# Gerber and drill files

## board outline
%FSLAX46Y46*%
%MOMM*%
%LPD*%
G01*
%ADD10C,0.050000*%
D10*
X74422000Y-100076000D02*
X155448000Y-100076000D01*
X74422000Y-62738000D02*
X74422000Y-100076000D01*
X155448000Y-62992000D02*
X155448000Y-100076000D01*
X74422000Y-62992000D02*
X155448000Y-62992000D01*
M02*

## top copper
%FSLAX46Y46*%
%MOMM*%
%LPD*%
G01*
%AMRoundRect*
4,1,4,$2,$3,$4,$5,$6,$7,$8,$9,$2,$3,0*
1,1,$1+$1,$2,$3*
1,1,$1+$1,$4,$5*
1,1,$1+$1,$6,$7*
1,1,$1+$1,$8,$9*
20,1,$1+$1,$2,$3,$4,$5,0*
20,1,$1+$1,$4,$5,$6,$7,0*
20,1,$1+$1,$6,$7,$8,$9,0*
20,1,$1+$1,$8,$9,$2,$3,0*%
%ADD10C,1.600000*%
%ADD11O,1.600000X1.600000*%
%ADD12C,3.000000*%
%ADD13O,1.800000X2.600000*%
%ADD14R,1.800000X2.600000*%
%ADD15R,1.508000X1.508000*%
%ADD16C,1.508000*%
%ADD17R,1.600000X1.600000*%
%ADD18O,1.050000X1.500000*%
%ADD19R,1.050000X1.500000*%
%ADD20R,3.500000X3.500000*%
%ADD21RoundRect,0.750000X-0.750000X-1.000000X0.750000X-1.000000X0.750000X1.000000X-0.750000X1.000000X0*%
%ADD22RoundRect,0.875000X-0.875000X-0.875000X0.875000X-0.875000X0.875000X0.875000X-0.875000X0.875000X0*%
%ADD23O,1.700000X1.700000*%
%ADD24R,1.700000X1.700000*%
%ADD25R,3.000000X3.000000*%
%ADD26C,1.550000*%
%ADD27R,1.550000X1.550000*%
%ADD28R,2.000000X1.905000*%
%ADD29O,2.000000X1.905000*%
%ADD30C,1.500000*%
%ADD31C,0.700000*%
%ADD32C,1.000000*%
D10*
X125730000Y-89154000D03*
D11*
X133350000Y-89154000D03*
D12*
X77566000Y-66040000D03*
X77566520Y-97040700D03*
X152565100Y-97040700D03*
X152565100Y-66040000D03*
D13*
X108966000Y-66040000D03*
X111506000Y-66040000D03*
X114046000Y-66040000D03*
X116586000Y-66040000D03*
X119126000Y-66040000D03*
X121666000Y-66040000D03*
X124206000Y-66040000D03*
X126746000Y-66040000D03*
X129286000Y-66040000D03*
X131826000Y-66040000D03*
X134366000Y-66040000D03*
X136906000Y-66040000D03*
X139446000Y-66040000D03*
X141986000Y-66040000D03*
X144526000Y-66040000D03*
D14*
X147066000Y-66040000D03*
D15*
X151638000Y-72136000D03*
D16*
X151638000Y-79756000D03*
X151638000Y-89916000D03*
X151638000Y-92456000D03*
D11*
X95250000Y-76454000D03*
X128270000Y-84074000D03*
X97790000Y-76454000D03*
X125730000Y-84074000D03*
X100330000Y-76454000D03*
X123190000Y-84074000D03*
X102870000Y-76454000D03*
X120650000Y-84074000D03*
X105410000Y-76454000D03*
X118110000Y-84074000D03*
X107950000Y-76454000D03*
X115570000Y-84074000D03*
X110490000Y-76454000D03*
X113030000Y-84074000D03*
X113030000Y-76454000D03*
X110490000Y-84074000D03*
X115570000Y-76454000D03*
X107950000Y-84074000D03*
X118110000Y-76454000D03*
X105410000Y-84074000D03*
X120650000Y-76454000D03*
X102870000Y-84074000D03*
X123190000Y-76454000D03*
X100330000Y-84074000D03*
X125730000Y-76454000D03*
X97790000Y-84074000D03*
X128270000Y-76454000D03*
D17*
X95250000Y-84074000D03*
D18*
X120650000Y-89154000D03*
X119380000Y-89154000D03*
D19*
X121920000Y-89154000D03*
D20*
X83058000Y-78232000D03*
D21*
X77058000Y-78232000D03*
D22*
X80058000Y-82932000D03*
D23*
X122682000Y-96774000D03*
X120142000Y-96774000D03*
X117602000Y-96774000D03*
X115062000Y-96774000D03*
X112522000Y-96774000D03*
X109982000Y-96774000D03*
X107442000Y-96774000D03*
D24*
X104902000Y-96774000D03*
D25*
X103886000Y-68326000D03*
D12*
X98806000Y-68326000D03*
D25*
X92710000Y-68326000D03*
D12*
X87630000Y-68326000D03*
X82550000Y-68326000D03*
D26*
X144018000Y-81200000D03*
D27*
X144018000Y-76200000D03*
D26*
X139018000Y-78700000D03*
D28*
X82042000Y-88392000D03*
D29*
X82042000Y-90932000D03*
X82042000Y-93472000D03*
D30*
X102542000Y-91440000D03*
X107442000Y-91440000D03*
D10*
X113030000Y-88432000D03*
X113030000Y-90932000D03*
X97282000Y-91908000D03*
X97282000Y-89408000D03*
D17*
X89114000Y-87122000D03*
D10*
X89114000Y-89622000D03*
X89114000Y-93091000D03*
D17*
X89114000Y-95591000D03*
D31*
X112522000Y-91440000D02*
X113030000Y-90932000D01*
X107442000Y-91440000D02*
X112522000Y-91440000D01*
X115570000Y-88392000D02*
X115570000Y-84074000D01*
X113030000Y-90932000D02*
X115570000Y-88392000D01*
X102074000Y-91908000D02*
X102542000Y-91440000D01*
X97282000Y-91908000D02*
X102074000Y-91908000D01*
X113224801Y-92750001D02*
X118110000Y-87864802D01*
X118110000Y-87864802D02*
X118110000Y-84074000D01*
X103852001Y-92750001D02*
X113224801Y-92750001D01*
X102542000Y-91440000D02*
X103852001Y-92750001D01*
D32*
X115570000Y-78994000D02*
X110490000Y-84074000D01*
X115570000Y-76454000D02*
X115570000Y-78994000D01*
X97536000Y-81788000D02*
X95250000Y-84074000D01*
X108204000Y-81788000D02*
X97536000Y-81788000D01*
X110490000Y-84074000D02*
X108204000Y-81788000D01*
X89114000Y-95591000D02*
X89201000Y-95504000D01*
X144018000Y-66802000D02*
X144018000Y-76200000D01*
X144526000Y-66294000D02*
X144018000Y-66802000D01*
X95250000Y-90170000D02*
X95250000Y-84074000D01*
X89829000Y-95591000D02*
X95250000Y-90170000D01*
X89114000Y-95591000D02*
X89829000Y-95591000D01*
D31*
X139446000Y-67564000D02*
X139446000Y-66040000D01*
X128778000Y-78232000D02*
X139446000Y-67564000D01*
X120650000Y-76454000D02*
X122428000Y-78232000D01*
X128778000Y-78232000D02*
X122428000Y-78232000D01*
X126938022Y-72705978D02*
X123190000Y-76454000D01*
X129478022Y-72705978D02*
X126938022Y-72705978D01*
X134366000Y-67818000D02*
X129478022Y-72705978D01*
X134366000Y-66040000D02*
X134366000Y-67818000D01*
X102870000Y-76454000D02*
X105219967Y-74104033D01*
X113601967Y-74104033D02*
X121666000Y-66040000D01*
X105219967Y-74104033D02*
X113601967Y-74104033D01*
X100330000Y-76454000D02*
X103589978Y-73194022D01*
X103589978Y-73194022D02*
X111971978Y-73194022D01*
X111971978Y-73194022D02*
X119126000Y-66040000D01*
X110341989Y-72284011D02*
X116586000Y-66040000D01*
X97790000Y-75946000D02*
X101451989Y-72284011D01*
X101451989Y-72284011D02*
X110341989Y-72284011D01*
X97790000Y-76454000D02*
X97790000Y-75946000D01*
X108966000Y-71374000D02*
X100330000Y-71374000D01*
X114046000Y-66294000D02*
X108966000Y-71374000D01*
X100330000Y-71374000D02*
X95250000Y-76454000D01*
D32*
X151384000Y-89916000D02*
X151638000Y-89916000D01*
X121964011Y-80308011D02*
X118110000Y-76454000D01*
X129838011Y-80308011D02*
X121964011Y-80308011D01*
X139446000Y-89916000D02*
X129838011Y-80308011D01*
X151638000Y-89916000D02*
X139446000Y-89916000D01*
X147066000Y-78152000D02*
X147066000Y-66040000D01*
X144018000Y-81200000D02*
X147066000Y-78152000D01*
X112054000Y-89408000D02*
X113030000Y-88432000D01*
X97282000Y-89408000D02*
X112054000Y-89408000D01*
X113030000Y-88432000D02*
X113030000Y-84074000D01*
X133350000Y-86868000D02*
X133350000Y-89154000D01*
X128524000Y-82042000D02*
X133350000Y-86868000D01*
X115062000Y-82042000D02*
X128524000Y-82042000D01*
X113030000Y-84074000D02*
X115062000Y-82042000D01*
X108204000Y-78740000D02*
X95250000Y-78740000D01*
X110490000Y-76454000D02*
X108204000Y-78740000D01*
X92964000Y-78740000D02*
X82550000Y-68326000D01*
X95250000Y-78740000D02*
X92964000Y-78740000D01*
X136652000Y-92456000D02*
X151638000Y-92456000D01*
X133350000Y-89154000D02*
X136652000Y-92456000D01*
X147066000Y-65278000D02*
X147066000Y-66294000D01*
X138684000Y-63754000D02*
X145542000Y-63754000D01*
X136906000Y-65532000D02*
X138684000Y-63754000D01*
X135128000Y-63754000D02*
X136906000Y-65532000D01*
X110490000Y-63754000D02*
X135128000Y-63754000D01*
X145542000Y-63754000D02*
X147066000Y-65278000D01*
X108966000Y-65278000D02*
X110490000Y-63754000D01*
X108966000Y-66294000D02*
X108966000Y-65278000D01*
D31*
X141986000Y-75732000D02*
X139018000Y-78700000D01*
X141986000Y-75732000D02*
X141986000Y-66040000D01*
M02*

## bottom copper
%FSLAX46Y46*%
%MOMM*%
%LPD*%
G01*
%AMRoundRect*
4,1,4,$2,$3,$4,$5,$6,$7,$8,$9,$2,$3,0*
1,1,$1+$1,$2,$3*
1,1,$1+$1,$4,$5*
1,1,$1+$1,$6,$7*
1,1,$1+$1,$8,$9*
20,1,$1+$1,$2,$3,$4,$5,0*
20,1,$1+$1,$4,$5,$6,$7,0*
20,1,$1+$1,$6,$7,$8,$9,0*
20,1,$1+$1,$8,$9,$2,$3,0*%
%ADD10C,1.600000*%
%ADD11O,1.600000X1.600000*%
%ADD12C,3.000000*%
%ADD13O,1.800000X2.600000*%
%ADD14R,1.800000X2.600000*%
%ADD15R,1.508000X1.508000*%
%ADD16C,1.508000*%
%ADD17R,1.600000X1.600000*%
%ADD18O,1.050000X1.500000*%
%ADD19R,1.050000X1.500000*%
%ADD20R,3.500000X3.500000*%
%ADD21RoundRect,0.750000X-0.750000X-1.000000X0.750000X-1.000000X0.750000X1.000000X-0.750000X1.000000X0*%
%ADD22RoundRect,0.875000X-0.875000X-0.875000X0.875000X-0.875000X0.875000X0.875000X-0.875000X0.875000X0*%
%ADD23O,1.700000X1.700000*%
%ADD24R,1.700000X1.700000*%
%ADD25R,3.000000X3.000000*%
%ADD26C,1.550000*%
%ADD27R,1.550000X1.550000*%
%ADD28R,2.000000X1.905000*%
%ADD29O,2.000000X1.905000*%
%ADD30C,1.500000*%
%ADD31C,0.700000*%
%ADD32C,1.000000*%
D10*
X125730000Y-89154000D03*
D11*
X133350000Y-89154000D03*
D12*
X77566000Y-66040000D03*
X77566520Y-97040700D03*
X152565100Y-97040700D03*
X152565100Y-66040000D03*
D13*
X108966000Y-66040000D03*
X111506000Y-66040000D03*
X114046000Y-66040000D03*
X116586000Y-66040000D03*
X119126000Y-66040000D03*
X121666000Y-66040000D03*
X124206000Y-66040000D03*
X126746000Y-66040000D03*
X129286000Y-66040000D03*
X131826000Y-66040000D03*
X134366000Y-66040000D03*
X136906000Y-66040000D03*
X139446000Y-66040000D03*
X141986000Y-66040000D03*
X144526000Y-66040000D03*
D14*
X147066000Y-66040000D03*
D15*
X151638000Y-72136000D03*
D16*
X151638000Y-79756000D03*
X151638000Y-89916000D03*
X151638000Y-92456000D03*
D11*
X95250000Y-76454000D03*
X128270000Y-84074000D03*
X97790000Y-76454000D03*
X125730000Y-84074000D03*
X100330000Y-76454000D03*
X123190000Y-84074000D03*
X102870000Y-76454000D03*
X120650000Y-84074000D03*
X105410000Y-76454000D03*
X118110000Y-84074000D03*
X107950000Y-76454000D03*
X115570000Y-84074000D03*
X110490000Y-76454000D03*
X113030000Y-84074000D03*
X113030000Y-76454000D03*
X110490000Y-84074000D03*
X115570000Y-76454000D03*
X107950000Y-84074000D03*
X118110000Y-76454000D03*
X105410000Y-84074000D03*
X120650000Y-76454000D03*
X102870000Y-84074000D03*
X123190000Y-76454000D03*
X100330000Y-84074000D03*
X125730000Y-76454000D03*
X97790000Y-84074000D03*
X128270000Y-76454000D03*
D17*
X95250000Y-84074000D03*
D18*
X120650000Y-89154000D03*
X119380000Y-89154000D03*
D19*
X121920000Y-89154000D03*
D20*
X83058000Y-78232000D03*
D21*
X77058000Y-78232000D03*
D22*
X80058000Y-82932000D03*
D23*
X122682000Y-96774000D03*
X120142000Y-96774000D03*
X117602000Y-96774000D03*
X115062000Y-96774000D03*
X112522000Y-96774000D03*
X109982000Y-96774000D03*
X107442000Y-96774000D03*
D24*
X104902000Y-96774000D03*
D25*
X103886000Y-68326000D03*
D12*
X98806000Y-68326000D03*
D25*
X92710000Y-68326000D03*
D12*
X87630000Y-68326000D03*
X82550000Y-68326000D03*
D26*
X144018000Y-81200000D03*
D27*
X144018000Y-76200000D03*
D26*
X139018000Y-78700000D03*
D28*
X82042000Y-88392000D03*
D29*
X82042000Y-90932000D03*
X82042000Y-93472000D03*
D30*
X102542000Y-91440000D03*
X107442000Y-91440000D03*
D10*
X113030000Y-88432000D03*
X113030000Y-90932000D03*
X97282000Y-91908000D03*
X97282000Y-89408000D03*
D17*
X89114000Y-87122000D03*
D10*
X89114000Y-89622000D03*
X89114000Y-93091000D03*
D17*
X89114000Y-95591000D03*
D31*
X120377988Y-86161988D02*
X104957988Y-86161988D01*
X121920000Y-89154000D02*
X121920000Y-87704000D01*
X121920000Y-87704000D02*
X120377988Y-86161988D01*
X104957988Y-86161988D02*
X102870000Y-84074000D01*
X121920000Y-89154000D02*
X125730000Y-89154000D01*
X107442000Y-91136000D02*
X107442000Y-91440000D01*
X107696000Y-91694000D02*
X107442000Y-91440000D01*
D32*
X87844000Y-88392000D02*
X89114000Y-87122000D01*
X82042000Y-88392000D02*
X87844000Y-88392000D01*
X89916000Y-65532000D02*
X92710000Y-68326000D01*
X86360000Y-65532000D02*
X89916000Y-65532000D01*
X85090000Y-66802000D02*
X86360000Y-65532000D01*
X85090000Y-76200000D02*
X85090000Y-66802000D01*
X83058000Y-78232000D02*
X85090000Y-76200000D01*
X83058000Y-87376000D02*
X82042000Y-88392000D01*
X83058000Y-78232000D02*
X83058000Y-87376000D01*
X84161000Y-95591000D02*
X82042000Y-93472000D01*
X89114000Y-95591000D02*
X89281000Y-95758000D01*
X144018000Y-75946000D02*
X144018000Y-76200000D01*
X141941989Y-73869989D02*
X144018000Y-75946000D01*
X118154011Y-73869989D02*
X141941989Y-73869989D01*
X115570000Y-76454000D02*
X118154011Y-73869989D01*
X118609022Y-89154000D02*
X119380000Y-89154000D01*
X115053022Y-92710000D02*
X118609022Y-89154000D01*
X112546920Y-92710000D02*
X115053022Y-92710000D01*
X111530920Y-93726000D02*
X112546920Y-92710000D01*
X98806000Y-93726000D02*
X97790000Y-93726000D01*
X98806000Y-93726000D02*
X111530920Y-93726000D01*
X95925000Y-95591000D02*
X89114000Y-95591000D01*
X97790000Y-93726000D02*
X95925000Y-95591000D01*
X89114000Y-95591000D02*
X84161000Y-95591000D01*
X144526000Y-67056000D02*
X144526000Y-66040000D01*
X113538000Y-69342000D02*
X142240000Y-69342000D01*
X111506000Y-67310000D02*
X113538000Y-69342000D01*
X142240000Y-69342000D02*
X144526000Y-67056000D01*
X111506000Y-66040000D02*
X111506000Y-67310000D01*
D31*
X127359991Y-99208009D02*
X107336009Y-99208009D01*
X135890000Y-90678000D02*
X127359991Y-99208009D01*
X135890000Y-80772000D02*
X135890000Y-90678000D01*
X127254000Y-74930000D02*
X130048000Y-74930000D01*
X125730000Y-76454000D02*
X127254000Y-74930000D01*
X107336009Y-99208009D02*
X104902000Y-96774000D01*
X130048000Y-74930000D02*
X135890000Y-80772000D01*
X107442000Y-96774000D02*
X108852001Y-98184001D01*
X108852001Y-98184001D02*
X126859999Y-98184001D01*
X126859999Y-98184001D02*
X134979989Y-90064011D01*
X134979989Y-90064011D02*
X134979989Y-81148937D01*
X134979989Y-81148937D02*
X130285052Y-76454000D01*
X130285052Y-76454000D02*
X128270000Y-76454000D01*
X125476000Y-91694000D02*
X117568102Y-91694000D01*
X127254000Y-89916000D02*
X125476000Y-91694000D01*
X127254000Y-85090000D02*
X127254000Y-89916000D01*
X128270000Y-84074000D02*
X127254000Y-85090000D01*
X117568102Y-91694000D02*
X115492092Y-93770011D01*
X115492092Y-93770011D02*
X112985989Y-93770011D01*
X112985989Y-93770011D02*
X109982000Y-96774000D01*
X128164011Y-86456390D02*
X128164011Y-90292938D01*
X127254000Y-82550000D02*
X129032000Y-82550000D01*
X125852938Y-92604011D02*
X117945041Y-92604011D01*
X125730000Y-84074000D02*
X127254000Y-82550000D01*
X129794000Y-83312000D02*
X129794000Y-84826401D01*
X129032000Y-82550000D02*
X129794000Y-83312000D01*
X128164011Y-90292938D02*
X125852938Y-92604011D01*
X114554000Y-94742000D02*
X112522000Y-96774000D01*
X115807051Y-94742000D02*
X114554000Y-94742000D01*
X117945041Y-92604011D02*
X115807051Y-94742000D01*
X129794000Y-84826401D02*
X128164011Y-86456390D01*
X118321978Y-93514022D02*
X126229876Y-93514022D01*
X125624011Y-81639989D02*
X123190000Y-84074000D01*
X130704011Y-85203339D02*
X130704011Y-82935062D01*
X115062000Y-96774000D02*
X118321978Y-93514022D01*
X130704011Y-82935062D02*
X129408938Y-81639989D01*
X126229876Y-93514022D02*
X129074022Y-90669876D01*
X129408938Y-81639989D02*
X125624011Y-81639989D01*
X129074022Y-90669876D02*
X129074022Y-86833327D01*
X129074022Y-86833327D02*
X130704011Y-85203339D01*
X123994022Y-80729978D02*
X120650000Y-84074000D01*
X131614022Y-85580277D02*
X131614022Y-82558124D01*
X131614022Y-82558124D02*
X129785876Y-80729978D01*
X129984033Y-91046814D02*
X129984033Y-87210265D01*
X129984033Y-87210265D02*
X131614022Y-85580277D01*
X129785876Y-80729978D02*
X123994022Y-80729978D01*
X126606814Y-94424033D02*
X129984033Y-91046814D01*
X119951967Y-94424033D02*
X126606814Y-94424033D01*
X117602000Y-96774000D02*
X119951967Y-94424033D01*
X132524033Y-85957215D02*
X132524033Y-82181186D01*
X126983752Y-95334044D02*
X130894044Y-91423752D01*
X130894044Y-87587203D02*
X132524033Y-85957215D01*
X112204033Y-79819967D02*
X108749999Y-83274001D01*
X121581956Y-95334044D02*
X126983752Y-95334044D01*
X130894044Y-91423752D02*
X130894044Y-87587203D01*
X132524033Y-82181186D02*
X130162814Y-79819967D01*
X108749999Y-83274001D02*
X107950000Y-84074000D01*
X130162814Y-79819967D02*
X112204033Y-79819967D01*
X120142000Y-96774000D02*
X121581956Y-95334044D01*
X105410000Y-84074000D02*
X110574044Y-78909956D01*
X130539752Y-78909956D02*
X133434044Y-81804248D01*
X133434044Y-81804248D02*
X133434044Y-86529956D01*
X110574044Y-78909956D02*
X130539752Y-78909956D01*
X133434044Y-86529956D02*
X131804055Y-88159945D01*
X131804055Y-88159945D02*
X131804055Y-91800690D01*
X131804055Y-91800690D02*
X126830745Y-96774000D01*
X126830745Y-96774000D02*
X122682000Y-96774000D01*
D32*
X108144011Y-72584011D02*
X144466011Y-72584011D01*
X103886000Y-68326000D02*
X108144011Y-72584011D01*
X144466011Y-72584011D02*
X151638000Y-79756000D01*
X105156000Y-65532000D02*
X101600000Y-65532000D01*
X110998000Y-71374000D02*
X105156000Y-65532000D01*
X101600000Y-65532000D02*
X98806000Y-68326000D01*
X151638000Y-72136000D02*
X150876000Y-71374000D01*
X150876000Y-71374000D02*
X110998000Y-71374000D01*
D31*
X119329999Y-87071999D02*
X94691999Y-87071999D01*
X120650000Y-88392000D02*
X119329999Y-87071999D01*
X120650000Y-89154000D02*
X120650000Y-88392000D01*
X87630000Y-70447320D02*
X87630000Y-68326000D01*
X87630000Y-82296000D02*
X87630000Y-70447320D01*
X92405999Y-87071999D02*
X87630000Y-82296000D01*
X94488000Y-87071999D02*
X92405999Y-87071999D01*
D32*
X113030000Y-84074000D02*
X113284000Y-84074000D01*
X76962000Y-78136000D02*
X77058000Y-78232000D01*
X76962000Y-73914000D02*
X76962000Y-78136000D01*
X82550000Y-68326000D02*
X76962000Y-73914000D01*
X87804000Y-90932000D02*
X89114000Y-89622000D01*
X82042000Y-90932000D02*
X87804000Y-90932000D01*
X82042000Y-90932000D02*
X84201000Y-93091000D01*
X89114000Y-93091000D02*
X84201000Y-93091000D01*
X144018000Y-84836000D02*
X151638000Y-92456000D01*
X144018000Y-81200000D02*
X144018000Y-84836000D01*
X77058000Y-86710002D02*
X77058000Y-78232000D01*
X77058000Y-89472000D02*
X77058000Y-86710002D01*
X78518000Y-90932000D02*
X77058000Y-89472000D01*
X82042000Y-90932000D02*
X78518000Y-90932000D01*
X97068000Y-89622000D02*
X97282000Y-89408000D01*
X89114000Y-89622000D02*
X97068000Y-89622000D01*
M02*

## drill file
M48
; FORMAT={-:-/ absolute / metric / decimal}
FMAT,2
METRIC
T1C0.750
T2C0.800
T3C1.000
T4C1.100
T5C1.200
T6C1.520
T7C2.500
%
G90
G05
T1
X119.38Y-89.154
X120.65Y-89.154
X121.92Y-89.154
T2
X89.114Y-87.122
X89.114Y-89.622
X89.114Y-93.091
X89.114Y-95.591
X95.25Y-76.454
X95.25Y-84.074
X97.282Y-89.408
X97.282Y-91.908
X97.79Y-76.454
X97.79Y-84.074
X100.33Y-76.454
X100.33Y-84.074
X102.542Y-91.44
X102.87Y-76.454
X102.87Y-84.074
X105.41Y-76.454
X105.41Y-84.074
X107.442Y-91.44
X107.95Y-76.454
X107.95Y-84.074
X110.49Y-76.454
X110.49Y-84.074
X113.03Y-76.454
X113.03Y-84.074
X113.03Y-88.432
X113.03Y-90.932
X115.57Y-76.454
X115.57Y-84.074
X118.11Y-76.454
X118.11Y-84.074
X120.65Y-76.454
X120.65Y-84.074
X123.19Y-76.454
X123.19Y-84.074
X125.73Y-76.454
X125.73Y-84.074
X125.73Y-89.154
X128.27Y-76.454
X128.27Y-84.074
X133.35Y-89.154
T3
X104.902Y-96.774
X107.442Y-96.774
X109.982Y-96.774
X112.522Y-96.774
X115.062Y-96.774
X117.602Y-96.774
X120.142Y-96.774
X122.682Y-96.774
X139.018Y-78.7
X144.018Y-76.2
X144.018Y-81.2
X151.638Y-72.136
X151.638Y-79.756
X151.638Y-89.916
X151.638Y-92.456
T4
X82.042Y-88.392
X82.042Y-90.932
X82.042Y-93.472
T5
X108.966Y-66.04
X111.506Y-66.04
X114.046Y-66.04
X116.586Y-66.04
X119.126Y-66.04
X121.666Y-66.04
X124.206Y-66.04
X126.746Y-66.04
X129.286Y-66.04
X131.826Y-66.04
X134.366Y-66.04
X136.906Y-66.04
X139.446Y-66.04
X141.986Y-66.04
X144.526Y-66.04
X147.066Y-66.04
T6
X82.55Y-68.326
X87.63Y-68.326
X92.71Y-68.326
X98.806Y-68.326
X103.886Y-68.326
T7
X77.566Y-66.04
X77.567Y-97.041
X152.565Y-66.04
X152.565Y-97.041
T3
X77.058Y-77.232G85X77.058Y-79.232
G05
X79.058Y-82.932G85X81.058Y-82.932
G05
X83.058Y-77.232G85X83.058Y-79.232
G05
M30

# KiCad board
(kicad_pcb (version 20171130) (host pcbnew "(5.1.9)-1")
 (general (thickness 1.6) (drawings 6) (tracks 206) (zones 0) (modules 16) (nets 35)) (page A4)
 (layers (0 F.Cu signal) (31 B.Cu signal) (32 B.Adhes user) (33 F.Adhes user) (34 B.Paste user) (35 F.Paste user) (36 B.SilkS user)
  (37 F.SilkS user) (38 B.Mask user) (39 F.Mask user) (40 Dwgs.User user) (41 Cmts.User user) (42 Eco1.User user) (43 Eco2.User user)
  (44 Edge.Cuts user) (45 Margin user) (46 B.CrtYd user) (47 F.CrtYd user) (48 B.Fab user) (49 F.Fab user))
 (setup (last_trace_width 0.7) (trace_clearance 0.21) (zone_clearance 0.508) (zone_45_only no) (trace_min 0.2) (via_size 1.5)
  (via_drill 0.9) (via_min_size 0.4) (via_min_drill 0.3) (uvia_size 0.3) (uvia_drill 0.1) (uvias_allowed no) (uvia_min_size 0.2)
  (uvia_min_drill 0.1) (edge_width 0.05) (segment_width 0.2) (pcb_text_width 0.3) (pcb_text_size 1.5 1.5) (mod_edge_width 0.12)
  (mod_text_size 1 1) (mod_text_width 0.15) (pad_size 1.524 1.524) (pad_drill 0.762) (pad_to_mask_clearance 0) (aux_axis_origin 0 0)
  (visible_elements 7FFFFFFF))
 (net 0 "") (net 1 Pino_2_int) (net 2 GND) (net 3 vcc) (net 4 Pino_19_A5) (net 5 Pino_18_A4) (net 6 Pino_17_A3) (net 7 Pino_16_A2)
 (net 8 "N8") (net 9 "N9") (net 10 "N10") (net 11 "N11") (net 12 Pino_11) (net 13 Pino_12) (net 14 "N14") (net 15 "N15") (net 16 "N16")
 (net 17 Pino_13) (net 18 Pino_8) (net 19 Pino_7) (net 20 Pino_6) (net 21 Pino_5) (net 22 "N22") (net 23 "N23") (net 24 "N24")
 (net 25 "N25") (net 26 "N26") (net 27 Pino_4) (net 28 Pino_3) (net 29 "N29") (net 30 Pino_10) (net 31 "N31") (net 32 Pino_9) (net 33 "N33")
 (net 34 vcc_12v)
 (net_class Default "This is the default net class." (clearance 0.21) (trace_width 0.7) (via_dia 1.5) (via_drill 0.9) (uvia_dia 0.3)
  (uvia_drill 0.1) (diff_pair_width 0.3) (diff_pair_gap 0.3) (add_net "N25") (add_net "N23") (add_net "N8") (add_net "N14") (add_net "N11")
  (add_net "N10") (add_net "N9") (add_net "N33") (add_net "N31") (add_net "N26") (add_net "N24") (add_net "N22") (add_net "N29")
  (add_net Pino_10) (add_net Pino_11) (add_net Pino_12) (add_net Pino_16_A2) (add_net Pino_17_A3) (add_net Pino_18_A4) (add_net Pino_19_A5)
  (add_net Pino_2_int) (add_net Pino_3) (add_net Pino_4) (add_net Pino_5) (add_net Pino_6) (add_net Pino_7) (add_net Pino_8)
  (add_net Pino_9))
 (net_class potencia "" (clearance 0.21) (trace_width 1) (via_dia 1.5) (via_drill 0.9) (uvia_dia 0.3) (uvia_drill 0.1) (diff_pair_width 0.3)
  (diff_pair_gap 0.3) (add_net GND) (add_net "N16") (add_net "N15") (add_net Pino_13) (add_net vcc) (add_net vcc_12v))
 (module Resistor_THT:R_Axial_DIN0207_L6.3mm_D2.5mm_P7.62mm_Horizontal (layer F.Cu) (at 125.73 89.154)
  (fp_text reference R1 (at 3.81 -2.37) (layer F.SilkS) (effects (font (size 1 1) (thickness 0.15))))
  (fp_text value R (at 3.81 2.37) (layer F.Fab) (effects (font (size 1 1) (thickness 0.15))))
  (pad 1 thru_hole circle (at 0 0) (size 1.6 1.6) (drill 0.8) (layers *.Cu *.Mask) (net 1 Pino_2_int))
  (pad 2 thru_hole oval (at 7.62 0) (size 1.6 1.6) (drill 0.8) (layers *.Cu *.Mask) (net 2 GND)))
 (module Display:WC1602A (layer B.Cu) (at 147.066 66.04 180)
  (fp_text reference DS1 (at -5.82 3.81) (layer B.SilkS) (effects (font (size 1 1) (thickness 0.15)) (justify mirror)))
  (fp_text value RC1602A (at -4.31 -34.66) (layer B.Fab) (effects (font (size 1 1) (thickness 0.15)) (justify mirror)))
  (pad "" thru_hole circle (at 69.5 0 180) (size 3 3) (drill 2.5) (layers *.Cu *.Mask))
  (pad "" thru_hole circle (at 69.49948 -31.0007 180) (size 3 3) (drill 2.5) (layers *.Cu *.Mask))
  (pad "" thru_hole circle (at -5.4991 -31.0007 180) (size 3 3) (drill 2.5) (layers *.Cu *.Mask))
  (pad "" thru_hole circle (at -5.4991 0 180) (size 3 3) (drill 2.5) (layers *.Cu *.Mask))
  (pad 16 thru_hole oval (at 38.1 0 180) (size 1.8 2.6) (drill 1.2) (layers *.Cu *.Mask) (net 2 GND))
  (pad 15 thru_hole oval (at 35.56 0 180) (size 1.8 2.6) (drill 1.2) (layers *.Cu *.Mask) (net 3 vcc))
  (pad 14 thru_hole oval (at 33.02 0 180) (size 1.8 2.6) (drill 1.2) (layers *.Cu *.Mask) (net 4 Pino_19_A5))
  (pad 13 thru_hole oval (at 30.48 0 180) (size 1.8 2.6) (drill 1.2) (layers *.Cu *.Mask) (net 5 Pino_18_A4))
  (pad 12 thru_hole oval (at 27.94 0 180) (size 1.8 2.6) (drill 1.2) (layers *.Cu *.Mask) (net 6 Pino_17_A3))
  (pad 11 thru_hole oval (at 25.4 0 180) (size 1.8 2.6) (drill 1.2) (layers *.Cu *.Mask) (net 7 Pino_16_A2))
  (pad 10 thru_hole oval (at 22.86 0 180) (size 1.8 2.6) (drill 1.2) (layers *.Cu *.Mask) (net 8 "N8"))
  (pad 9 thru_hole oval (at 20.32 0 180) (size 1.8 2.6) (drill 1.2) (layers *.Cu *.Mask) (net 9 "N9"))
  (pad 8 thru_hole oval (at 17.78 0 180) (size 1.8 2.6) (drill 1.2) (layers *.Cu *.Mask) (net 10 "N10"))
  (pad 7 thru_hole oval (at 15.24 0 180) (size 1.8 2.6) (drill 1.2) (layers *.Cu *.Mask) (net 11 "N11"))
  (pad 6 thru_hole oval (at 12.7 0 180) (size 1.8 2.6) (drill 1.2) (layers *.Cu *.Mask) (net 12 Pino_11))
  (pad 5 thru_hole oval (at 10.16 0 180) (size 1.8 2.6) (drill 1.2) (layers *.Cu *.Mask) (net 2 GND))
  (pad 4 thru_hole oval (at 7.62 0 180) (size 1.8 2.6) (drill 1.2) (layers *.Cu *.Mask) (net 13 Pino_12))
  (pad 3 thru_hole oval (at 5.08 0 180) (size 1.8 2.6) (drill 1.2) (layers *.Cu *.Mask) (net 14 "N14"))
  (pad 2 thru_hole oval (at 2.54 0 180) (size 1.8 2.6) (drill 1.2) (layers *.Cu *.Mask) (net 3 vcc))
  (pad 1 thru_hole rect (at 0 0 180) (size 1.8 2.6) (drill 1.2) (layers *.Cu *.Mask) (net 2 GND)))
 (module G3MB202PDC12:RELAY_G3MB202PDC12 (layer F.Cu) (at 150.238 82.296 270)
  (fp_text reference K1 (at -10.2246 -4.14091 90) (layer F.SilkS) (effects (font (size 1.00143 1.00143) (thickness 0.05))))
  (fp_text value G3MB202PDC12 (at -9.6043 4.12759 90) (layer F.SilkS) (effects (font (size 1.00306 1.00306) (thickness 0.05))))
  (pad 1 thru_hole rect (at -10.16 -1.4 90) (size 1.508 1.508) (drill 1) (layers *.Cu *.Mask) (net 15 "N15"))
  (pad 2 thru_hole circle (at -2.54 -1.4 90) (size 1.508 1.508) (drill 1) (layers *.Cu *.Mask) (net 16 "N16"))
  (pad 3 thru_hole circle (at 7.62 -1.4 90) (size 1.508 1.508) (drill 1) (layers *.Cu *.Mask) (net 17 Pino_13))
  (pad 4 thru_hole circle (at 10.16 -1.4 90) (size 1.508 1.508) (drill 1) (layers *.Cu *.Mask) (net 2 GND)))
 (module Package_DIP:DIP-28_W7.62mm (layer F.Cu) (at 95.25 84.074 90)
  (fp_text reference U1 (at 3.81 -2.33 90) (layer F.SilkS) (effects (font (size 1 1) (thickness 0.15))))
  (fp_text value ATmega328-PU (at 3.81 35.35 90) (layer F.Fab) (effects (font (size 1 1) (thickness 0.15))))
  (pad 28 thru_hole oval (at 7.62 0 90) (size 1.6 1.6) (drill 0.8) (layers *.Cu *.Mask) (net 4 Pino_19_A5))
  (pad 14 thru_hole oval (at 0 33.02 90) (size 1.6 1.6) (drill 0.8) (layers *.Cu *.Mask) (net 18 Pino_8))
  (pad 27 thru_hole oval (at 7.62 2.54 90) (size 1.6 1.6) (drill 0.8) (layers *.Cu *.Mask) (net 5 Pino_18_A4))
  (pad 13 thru_hole oval (at 0 30.48 90) (size 1.6 1.6) (drill 0.8) (layers *.Cu *.Mask) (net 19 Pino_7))
  (pad 26 thru_hole oval (at 7.62 5.08 90) (size 1.6 1.6) (drill 0.8) (layers *.Cu *.Mask) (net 6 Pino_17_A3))
  (pad 12 thru_hole oval (at 0 27.94 90) (size 1.6 1.6) (drill 0.8) (layers *.Cu *.Mask) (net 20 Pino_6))
  (pad 25 thru_hole oval (at 7.62 7.62 90) (size 1.6 1.6) (drill 0.8) (layers *.Cu *.Mask) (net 7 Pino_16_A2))
  (pad 11 thru_hole oval (at 0 25.4 90) (size 1.6 1.6) (drill 0.8) (layers *.Cu *.Mask) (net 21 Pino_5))
  (pad 24 thru_hole oval (at 7.62 10.16 90) (size 1.6 1.6) (drill 0.8) (layers *.Cu *.Mask) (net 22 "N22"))
  (pad 10 thru_hole oval (at 0 22.86 90) (size 1.6 1.6) (drill 0.8) (layers *.Cu *.Mask) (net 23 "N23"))
  (pad 23 thru_hole oval (at 7.62 12.7 90) (size 1.6 1.6) (drill 0.8) (layers *.Cu *.Mask) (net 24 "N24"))
  (pad 9 thru_hole oval (at 0 20.32 90) (size 1.6 1.6) (drill 0.8) (layers *.Cu *.Mask) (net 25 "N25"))
  (pad 22 thru_hole oval (at 7.62 15.24 90) (size 1.6 1.6) (drill 0.8) (layers *.Cu *.Mask) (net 2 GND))
  (pad 8 thru_hole oval (at 0 17.78 90) (size 1.6 1.6) (drill 0.8) (layers *.Cu *.Mask) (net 2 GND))
  (pad 21 thru_hole oval (at 7.62 17.78 90) (size 1.6 1.6) (drill 0.8) (layers *.Cu *.Mask) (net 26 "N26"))
  (pad 7 thru_hole oval (at 0 15.24 90) (size 1.6 1.6) (drill 0.8) (layers *.Cu *.Mask) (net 3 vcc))
  (pad 20 thru_hole oval (at 7.62 20.32 90) (size 1.6 1.6) (drill 0.8) (layers *.Cu *.Mask) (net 3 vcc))
  (pad 6 thru_hole oval (at 0 12.7 90) (size 1.6 1.6) (drill 0.8) (layers *.Cu *.Mask) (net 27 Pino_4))
  (pad 19 thru_hole oval (at 7.62 22.86 90) (size 1.6 1.6) (drill 0.8) (layers *.Cu *.Mask) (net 17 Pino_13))
  (pad 5 thru_hole oval (at 0 10.16 90) (size 1.6 1.6) (drill 0.8) (layers *.Cu *.Mask) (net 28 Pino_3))
  (pad 18 thru_hole oval (at 7.62 25.4 90) (size 1.6 1.6) (drill 0.8) (layers *.Cu *.Mask) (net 13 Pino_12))
  (pad 4 thru_hole oval (at 0 7.62 90) (size 1.6 1.6) (drill 0.8) (layers *.Cu *.Mask) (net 1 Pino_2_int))
  (pad 17 thru_hole oval (at 7.62 27.94 90) (size 1.6 1.6) (drill 0.8) (layers *.Cu *.Mask) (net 12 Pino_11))
  (pad 3 thru_hole oval (at 0 5.08 90) (size 1.6 1.6) (drill 0.8) (layers *.Cu *.Mask) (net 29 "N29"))
  (pad 16 thru_hole oval (at 7.62 30.48 90) (size 1.6 1.6) (drill 0.8) (layers *.Cu *.Mask) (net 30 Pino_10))
  (pad 2 thru_hole oval (at 0 2.54 90) (size 1.6 1.6) (drill 0.8) (layers *.Cu *.Mask) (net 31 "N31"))
  (pad 15 thru_hole oval (at 7.62 33.02 90) (size 1.6 1.6) (drill 0.8) (layers *.Cu *.Mask) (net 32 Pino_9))
  (pad 1 thru_hole rect (at 0 0 90) (size 1.6 1.6) (drill 0.8) (layers *.Cu *.Mask) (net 3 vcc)))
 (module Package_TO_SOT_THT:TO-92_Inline (layer F.Cu) (at 121.92 89.154 180)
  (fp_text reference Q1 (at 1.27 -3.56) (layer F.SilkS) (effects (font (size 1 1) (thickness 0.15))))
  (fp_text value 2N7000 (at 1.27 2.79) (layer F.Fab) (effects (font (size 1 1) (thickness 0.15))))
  (pad 2 thru_hole oval (at 1.27 0 180) (size 1.05 1.5) (drill 0.75) (layers *.Cu *.Mask) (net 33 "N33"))
  (pad 3 thru_hole oval (at 2.54 0 180) (size 1.05 1.5) (drill 0.75) (layers *.Cu *.Mask) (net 3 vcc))
  (pad 1 thru_hole rect (at 0 0 180) (size 1.05 1.5) (drill 0.75) (layers *.Cu *.Mask) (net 1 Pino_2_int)))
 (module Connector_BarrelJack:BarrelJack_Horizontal (layer F.Cu) (at 83.058 78.232)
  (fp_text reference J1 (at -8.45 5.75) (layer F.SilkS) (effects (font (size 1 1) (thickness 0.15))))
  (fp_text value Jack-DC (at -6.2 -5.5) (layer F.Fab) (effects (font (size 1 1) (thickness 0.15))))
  (pad 1 thru_hole rect (at 0 0) (size 3.5 3.5) (drill oval 1 3) (layers *.Cu *.Mask) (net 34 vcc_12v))
  (pad 2 thru_hole roundrect (at -6 0) (size 3 3.5) (drill oval 1 3) (layers *.Cu *.Mask) (roundrect_rratio 0.25) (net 2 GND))
  (pad 3 thru_hole roundrect (at -3 4.7) (size 3.5 3.5) (drill oval 3 1) (layers *.Cu *.Mask) (roundrect_rratio 0.25)))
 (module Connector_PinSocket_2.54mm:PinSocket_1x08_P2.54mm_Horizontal (layer F.Cu) (at 104.902 96.774 90)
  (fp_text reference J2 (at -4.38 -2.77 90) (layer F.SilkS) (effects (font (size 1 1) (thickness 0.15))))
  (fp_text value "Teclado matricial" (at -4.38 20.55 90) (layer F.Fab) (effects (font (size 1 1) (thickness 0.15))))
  (pad 8 thru_hole oval (at 0 17.78 90) (size 1.7 1.7) (drill 1) (layers *.Cu *.Mask) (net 28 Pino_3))
  (pad 7 thru_hole oval (at 0 15.24 90) (size 1.7 1.7) (drill 1) (layers *.Cu *.Mask) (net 27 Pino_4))
  (pad 6 thru_hole oval (at 0 12.7 90) (size 1.7 1.7) (drill 1) (layers *.Cu *.Mask) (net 21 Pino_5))
  (pad 5 thru_hole oval (at 0 10.16 90) (size 1.7 1.7) (drill 1) (layers *.Cu *.Mask) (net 20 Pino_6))
  (pad 4 thru_hole oval (at 0 7.62 90) (size 1.7 1.7) (drill 1) (layers *.Cu *.Mask) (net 19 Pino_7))
  (pad 3 thru_hole oval (at 0 5.08 90) (size 1.7 1.7) (drill 1) (layers *.Cu *.Mask) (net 18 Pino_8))
  (pad 2 thru_hole oval (at 0 2.54 90) (size 1.7 1.7) (drill 1) (layers *.Cu *.Mask) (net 32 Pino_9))
  (pad 1 thru_hole rect (at 0 0 90) (size 1.7 1.7) (drill 1) (layers *.Cu *.Mask) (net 30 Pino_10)))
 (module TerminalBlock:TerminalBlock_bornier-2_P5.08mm (layer F.Cu) (at 103.886 68.326 180)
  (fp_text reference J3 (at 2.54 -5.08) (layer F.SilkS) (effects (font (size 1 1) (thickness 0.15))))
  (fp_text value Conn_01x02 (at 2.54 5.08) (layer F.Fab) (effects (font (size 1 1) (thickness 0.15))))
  (pad 1 thru_hole rect (at 0 0 180) (size 3 3) (drill 1.52) (layers *.Cu *.Mask) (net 16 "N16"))
  (pad 2 thru_hole circle (at 5.08 0 180) (size 3 3) (drill 1.52) (layers *.Cu *.Mask) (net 15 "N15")))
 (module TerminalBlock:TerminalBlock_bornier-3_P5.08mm (layer F.Cu) (at 92.71 68.326 180)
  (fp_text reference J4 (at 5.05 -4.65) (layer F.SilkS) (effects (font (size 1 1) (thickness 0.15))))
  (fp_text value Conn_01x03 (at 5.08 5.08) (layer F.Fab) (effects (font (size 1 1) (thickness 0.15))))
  (pad 1 thru_hole rect (at 0 0 180) (size 3 3) (drill 1.52) (layers *.Cu *.Mask) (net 34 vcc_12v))
  (pad 2 thru_hole circle (at 5.08 0 180) (size 3 3) (drill 1.52) (layers *.Cu *.Mask) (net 33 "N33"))
  (pad 3 thru_hole circle (at 10.16 0 180) (size 3 3) (drill 1.52) (layers *.Cu *.Mask) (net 2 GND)))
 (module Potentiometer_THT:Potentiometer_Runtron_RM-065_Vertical (layer F.Cu) (at 144.018 76.2 270)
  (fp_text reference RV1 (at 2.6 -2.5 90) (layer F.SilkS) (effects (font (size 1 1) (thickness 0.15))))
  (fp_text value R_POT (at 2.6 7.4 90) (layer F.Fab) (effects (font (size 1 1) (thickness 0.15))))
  (pad 3 thru_hole circle (at 5 0 270) (size 1.55 1.55) (drill 1) (layers *.Cu *.Mask) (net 2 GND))
  (pad 1 thru_hole rect (at 0 0 270) (size 1.55 1.55) (drill 1) (layers *.Cu *.Mask) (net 3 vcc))
  (pad 2 thru_hole circle (at 2.5 5 270) (size 1.55 1.55) (drill 1) (layers *.Cu *.Mask) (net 14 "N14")))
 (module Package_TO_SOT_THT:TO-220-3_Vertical (layer F.Cu) (at 82.042 88.392 270)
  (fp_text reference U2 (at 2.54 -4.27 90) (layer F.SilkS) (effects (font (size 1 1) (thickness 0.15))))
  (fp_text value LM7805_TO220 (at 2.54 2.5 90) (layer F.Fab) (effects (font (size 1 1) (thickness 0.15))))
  (pad 1 thru_hole rect (at 0 0 270) (size 1.905 2) (drill 1.1) (layers *.Cu *.Mask) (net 34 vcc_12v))
  (pad 2 thru_hole oval (at 2.54 0 270) (size 1.905 2) (drill 1.1) (layers *.Cu *.Mask) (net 2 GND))
  (pad 3 thru_hole oval (at 5.08 0 270) (size 1.905 2) (drill 1.1) (layers *.Cu *.Mask) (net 3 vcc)))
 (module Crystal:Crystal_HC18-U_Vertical (layer F.Cu) (at 107.442 91.44 180)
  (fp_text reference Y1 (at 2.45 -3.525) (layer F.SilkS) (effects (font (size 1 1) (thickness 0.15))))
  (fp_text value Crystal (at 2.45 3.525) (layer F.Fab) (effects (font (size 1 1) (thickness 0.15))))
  (pad 2 thru_hole circle (at 4.9 0 180) (size 1.5 1.5) (drill 0.8) (layers *.Cu *.Mask) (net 23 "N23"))
  (pad 1 thru_hole circle (at 0 0 180) (size 1.5 1.5) (drill 0.8) (layers *.Cu *.Mask) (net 25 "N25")))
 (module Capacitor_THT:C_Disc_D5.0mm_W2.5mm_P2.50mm (layer F.Cu) (at 113.03 88.432 270)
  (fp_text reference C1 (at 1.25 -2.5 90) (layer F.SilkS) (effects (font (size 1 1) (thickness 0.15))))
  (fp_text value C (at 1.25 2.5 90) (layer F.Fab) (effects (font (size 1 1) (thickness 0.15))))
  (pad 1 thru_hole circle (at 0 0 270) (size 1.6 1.6) (drill 0.8) (layers *.Cu *.Mask) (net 2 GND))
  (pad 2 thru_hole circle (at 2.5 0 270) (size 1.6 1.6) (drill 0.8) (layers *.Cu *.Mask) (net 25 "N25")))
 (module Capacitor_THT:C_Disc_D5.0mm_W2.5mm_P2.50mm (layer F.Cu) (at 97.282 89.408 270)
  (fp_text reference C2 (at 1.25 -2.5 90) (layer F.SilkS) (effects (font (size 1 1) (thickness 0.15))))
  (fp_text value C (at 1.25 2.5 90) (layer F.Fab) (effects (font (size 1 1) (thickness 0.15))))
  (pad 2 thru_hole circle (at 2.5 0 270) (size 1.6 1.6) (drill 0.8) (layers *.Cu *.Mask) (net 23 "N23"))
  (pad 1 thru_hole circle (at 0 0 270) (size 1.6 1.6) (drill 0.8) (layers *.Cu *.Mask) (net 2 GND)))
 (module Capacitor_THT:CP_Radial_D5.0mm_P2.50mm (layer F.Cu) (at 89.114 87.122 270)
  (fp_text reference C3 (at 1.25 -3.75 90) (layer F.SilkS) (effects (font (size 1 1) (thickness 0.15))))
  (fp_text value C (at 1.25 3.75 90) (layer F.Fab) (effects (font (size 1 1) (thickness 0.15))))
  (pad 1 thru_hole rect (at 0 0 270) (size 1.6 1.6) (drill 0.8) (layers *.Cu *.Mask) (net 34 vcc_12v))
  (pad 2 thru_hole circle (at 2.5 0 270) (size 1.6 1.6) (drill 0.8) (layers *.Cu *.Mask) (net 2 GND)))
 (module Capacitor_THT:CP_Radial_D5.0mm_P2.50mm (layer F.Cu) (at 89.114 95.591 90)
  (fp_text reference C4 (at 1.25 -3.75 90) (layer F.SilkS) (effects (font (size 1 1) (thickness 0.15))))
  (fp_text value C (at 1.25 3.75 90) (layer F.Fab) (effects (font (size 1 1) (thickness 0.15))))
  (pad 2 thru_hole circle (at 2.5 0 90) (size 1.6 1.6) (drill 0.8) (layers *.Cu *.Mask) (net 2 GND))
  (pad 1 thru_hole rect (at 0 0 90) (size 1.6 1.6) (drill 0.8) (layers *.Cu *.Mask) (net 3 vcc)))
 (gr_line (start 74.422 100.076) (end 155.448 100.076) (layer Edge.Cuts) (width 0.05))
 (gr_line (start 74.422 62.738) (end 74.422 100.076) (layer Edge.Cuts) (width 0.05))
 (gr_line (start 155.448 62.992) (end 155.448 100.076) (layer Edge.Cuts) (width 0.05))
 (gr_line (start 74.422 62.992) (end 155.448 62.992) (layer Edge.Cuts) (width 0.05))
 (segment (start 120.377988 86.161988) (end 104.957988 86.161988) (width 0.7) (layer B.Cu) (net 1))
 (segment (start 121.92 89.154) (end 121.92 87.704) (width 0.7) (layer B.Cu) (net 1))
 (segment (start 121.92 87.704) (end 120.377988 86.161988) (width 0.7) (layer B.Cu) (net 1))
 (segment (start 104.957988 86.161988) (end 102.87 84.074) (width 0.7) (layer B.Cu) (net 1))
 (segment (start 121.92 89.154) (end 125.73 89.154) (width 0.7) (layer B.Cu) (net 1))
 (segment (start 107.442 91.136) (end 107.442 91.44) (width 0.7) (layer B.Cu) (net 25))
 (segment (start 107.696 91.694) (end 107.442 91.44) (width 0.7) (layer B.Cu) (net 25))
 (segment (start 112.522 91.44) (end 113.03 90.932) (width 0.7) (layer F.Cu) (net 25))
 (segment (start 107.442 91.44) (end 112.522 91.44) (width 0.7) (layer F.Cu) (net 25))
 (segment (start 115.57 88.392) (end 115.57 84.074) (width 0.7) (layer F.Cu) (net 25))
 (segment (start 113.03 90.932) (end 115.57 88.392) (width 0.7) (layer F.Cu) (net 25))
 (segment (start 102.074 91.908) (end 102.542 91.44) (width 0.7) (layer F.Cu) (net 23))
 (segment (start 97.282 91.908) (end 102.074 91.908) (width 0.7) (layer F.Cu) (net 23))
 (segment (start 113.224801 92.750001) (end 118.11 87.864802) (width 0.7) (layer F.Cu) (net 23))
 (segment (start 118.11 87.864802) (end 118.11 84.074) (width 0.7) (layer F.Cu) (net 23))
 (segment (start 103.852001 92.750001) (end 113.224801 92.750001) (width 0.7) (layer F.Cu) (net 23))
 (segment (start 102.542 91.44) (end 103.852001 92.750001) (width 0.7) (layer F.Cu) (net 23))
 (segment (start 87.844 88.392) (end 89.114 87.122) (width 1) (layer B.Cu) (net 34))
 (segment (start 82.042 88.392) (end 87.844 88.392) (width 1) (layer B.Cu) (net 34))
 (segment (start 89.916 65.532) (end 92.71 68.326) (width 1) (layer B.Cu) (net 34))
 (segment (start 86.36 65.532) (end 89.916 65.532) (width 1) (layer B.Cu) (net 34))
 (segment (start 85.09 66.802) (end 86.36 65.532) (width 1) (layer B.Cu) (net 34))
 (segment (start 85.09 76.2) (end 85.09 66.802) (width 1) (layer B.Cu) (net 34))
 (segment (start 83.058 78.232) (end 85.09 76.2) (width 1) (layer B.Cu) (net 34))
 (segment (start 83.058 87.376) (end 82.042 88.392) (width 1) (layer B.Cu) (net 34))
 (segment (start 83.058 78.232) (end 83.058 87.376) (width 1) (layer B.Cu) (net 34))
 (segment (start 115.57 78.994) (end 110.49 84.074) (width 1) (layer F.Cu) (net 3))
 (segment (start 115.57 76.454) (end 115.57 78.994) (width 1) (layer F.Cu) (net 3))
 (segment (start 97.536 81.788) (end 95.25 84.074) (width 1) (layer F.Cu) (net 3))
 (segment (start 108.204 81.788) (end 97.536 81.788) (width 1) (layer F.Cu) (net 3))
 (segment (start 110.49 84.074) (end 108.204 81.788) (width 1) (layer F.Cu) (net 3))
 (segment (start 84.161 95.591) (end 82.042 93.472) (width 1) (layer B.Cu) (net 3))
 (segment (start 89.114 95.591) (end 89.201 95.504) (width 1) (layer F.Cu) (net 3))
 (segment (start 89.114 95.591) (end 89.281 95.758) (width 1) (layer B.Cu) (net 3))
 (segment (start 144.018 75.946) (end 144.018 76.2) (width 1) (layer B.Cu) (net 3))
 (segment (start 141.941989 73.869989) (end 144.018 75.946) (width 1) (layer B.Cu) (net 3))
 (segment (start 118.154011 73.869989) (end 141.941989 73.869989) (width 1) (layer B.Cu) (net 3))
 (segment (start 115.57 76.454) (end 118.154011 73.869989) (width 1) (layer B.Cu) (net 3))
 (segment (start 144.018 66.802) (end 144.018 76.2) (width 1) (layer F.Cu) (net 3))
 (segment (start 144.526 66.294) (end 144.018 66.802) (width 1) (layer F.Cu) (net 3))
 (segment (start 95.25 90.17) (end 95.25 84.074) (width 1) (layer F.Cu) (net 3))
 (segment (start 89.829 95.591) (end 95.25 90.17) (width 1) (layer F.Cu) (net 3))
 (segment (start 89.114 95.591) (end 89.829 95.591) (width 1) (layer F.Cu) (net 3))
 (segment (start 118.609022 89.154) (end 119.38 89.154) (width 1) (layer B.Cu) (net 3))
 (segment (start 115.053022 92.71) (end 118.609022 89.154) (width 1) (layer B.Cu) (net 3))
 (segment (start 112.54692 92.71) (end 115.053022 92.71) (width 1) (layer B.Cu) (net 3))
 (segment (start 111.53092 93.726) (end 112.54692 92.71) (width 1) (layer B.Cu) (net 3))
 (segment (start 98.806 93.726) (end 97.79 93.726) (width 1) (layer B.Cu) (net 3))
 (segment (start 98.806 93.726) (end 111.53092 93.726) (width 1) (layer B.Cu) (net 3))
 (segment (start 95.925 95.591) (end 89.114 95.591) (width 1) (layer B.Cu) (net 3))
 (segment (start 97.79 93.726) (end 95.925 95.591) (width 1) (layer B.Cu) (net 3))
 (segment (start 89.114 95.591) (end 84.161 95.591) (width 1) (layer B.Cu) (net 3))
 (segment (start 144.526 67.056) (end 144.526 66.04) (width 1) (layer B.Cu) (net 3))
 (segment (start 113.538 69.342) (end 142.24 69.342) (width 1) (layer B.Cu) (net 3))
 (segment (start 111.506 67.31) (end 113.538 69.342) (width 1) (layer B.Cu) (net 3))
 (segment (start 142.24 69.342) (end 144.526 67.056) (width 1) (layer B.Cu) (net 3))
 (segment (start 111.506 66.04) (end 111.506 67.31) (width 1) (layer B.Cu) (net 3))
 (segment (start 139.446 67.564) (end 139.446 66.04) (width 0.7) (layer F.Cu) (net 13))
 (segment (start 128.778 78.232) (end 139.446 67.564) (width 0.7) (layer F.Cu) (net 13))
 (segment (start 120.65 76.454) (end 122.428 78.232) (width 0.7) (layer F.Cu) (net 13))
 (segment (start 128.778 78.232) (end 122.428 78.232) (width 0.7) (layer F.Cu) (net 13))
 (segment (start 126.938022 72.705978) (end 123.19 76.454) (width 0.7) (layer F.Cu) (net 12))
 (segment (start 129.478022 72.705978) (end 126.938022 72.705978) (width 0.7) (layer F.Cu) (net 12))
 (segment (start 134.366 67.818) (end 129.478022 72.705978) (width 0.7) (layer F.Cu) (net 12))
 (segment (start 134.366 66.04) (end 134.366 67.818) (width 0.7) (layer F.Cu) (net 12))
 (segment (start 102.87 76.454) (end 105.219967 74.104033) (width 0.7) (layer F.Cu) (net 7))
 (segment (start 113.601967 74.104033) (end 121.666 66.04) (width 0.7) (layer F.Cu) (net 7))
 (segment (start 105.219967 74.104033) (end 113.601967 74.104033) (width 0.7) (layer F.Cu) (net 7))
 (segment (start 100.33 76.454) (end 103.589978 73.194022) (width 0.7) (layer F.Cu) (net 6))
 (segment (start 103.589978 73.194022) (end 111.971978 73.194022) (width 0.7) (layer F.Cu) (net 6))
 (segment (start 111.971978 73.194022) (end 119.126 66.04) (width 0.7) (layer F.Cu) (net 6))
 (segment (start 110.341989 72.284011) (end 116.586 66.04) (width 0.7) (layer F.Cu) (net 5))
 (segment (start 97.79 75.946) (end 101.451989 72.284011) (width 0.7) (layer F.Cu) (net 5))
 (segment (start 101.451989 72.284011) (end 110.341989 72.284011) (width 0.7) (layer F.Cu) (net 5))
 (segment (start 97.79 76.454) (end 97.79 75.946) (width 0.7) (layer F.Cu) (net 5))
 (segment (start 108.966 71.374) (end 100.33 71.374) (width 0.7) (layer F.Cu) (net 4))
 (segment (start 114.046 66.294) (end 108.966 71.374) (width 0.7) (layer F.Cu) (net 4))
 (segment (start 100.33 71.374) (end 95.25 76.454) (width 0.7) (layer F.Cu) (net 4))
 (segment (start 127.359991 99.208009) (end 107.336009 99.208009) (width 0.7) (layer B.Cu) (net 30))
 (segment (start 135.89 90.678) (end 127.359991 99.208009) (width 0.7) (layer B.Cu) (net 30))
 (segment (start 135.89 80.772) (end 135.89 90.678) (width 0.7) (layer B.Cu) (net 30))
 (segment (start 127.254 74.93) (end 130.048 74.93) (width 0.7) (layer B.Cu) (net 30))
 (segment (start 125.73 76.454) (end 127.254 74.93) (width 0.7) (layer B.Cu) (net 30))
 (segment (start 107.336009 99.208009) (end 104.902 96.774) (width 0.7) (layer B.Cu) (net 30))
 (segment (start 130.048 74.93) (end 135.89 80.772) (width 0.7) (layer B.Cu) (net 30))
 (segment (start 107.442 96.774) (end 108.852001 98.184001) (width 0.7) (layer B.Cu) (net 32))
 (segment (start 108.852001 98.184001) (end 126.859999 98.184001) (width 0.7) (layer B.Cu) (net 32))
 (segment (start 126.859999 98.184001) (end 134.979989 90.064011) (width 0.7) (layer B.Cu) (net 32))
 (segment (start 134.979989 90.064011) (end 134.979989 81.148937) (width 0.7) (layer B.Cu) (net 32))
 (segment (start 134.979989 81.148937) (end 130.285052 76.454) (width 0.7) (layer B.Cu) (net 32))
 (segment (start 130.285052 76.454) (end 128.27 76.454) (width 0.7) (layer B.Cu) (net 32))
 (segment (start 125.476 91.694) (end 117.568102 91.694) (width 0.7) (layer B.Cu) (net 18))
 (segment (start 127.254 89.916) (end 125.476 91.694) (width 0.7) (layer B.Cu) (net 18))
 (segment (start 127.254 85.09) (end 127.254 89.916) (width 0.7) (layer B.Cu) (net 18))
 (segment (start 128.27 84.074) (end 127.254 85.09) (width 0.7) (layer B.Cu) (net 18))
 (segment (start 117.568102 91.694) (end 115.492092 93.770011) (width 0.7) (layer B.Cu) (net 18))
 (segment (start 115.492092 93.770011) (end 112.985989 93.770011) (width 0.7) (layer B.Cu) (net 18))
 (segment (start 112.985989 93.770011) (end 109.982 96.774) (width 0.7) (layer B.Cu) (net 18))
 (segment (start 128.164011 86.45639) (end 128.164011 90.292938) (width 0.7) (layer B.Cu) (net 19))
 (segment (start 127.254 82.55) (end 129.032 82.55) (width 0.7) (layer B.Cu) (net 19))
 (segment (start 125.852938 92.604011) (end 117.945041 92.604011) (width 0.7) (layer B.Cu) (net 19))
 (segment (start 125.73 84.074) (end 127.254 82.55) (width 0.7) (layer B.Cu) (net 19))
 (segment (start 129.794 83.312) (end 129.794 84.826401) (width 0.7) (layer B.Cu) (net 19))
 (segment (start 129.032 82.55) (end 129.794 83.312) (width 0.7) (layer B.Cu) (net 19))
 (segment (start 128.164011 90.292938) (end 125.852938 92.604011) (width 0.7) (layer B.Cu) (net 19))
 (segment (start 114.554 94.742) (end 112.522 96.774) (width 0.7) (layer B.Cu) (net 19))
 (segment (start 115.807051 94.742) (end 114.554 94.742) (width 0.7) (layer B.Cu) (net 19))
 (segment (start 117.945041 92.604011) (end 115.807051 94.742) (width 0.7) (layer B.Cu) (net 19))
 (segment (start 129.794 84.826401) (end 128.164011 86.45639) (width 0.7) (layer B.Cu) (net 19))
 (segment (start 118.321978 93.514022) (end 126.229876 93.514022) (width 0.7) (layer B.Cu) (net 20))
 (segment (start 125.624011 81.639989) (end 123.19 84.074) (width 0.7) (layer B.Cu) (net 20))
 (segment (start 130.704011 85.203339) (end 130.704011 82.935062) (width 0.7) (layer B.Cu) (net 20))
 (segment (start 115.062 96.774) (end 118.321978 93.514022) (width 0.7) (layer B.Cu) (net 20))
 (segment (start 130.704011 82.935062) (end 129.408938 81.639989) (width 0.7) (layer B.Cu) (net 20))
 (segment (start 126.229876 93.514022) (end 129.074022 90.669876) (width 0.7) (layer B.Cu) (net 20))
 (segment (start 129.408938 81.639989) (end 125.624011 81.639989) (width 0.7) (layer B.Cu) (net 20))
 (segment (start 129.074022 90.669876) (end 129.074022 86.833327) (width 0.7) (layer B.Cu) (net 20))
 (segment (start 129.074022 86.833327) (end 130.704011 85.203339) (width 0.7) (layer B.Cu) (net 20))
 (segment (start 123.994022 80.729978) (end 120.65 84.074) (width 0.7) (layer B.Cu) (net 21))
 (segment (start 131.614022 85.580277) (end 131.614022 82.558124) (width 0.7) (layer B.Cu) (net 21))
 (segment (start 131.614022 82.558124) (end 129.785876 80.729978) (width 0.7) (layer B.Cu) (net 21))
 (segment (start 129.984033 91.046814) (end 129.984033 87.210265) (width 0.7) (layer B.Cu) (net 21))
 (segment (start 129.984033 87.210265) (end 131.614022 85.580277) (width 0.7) (layer B.Cu) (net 21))
 (segment (start 129.785876 80.729978) (end 123.994022 80.729978) (width 0.7) (layer B.Cu) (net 21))
 (segment (start 126.606814 94.424033) (end 129.984033 91.046814) (width 0.7) (layer B.Cu) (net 21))
 (segment (start 119.951967 94.424033) (end 126.606814 94.424033) (width 0.7) (layer B.Cu) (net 21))
 (segment (start 117.602 96.774) (end 119.951967 94.424033) (width 0.7) (layer B.Cu) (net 21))
 (segment (start 132.524033 85.957215) (end 132.524033 82.181186) (width 0.7) (layer B.Cu) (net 27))
 (segment (start 126.983752 95.334044) (end 130.894044 91.423752) (width 0.7) (layer B.Cu) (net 27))
 (segment (start 130.894044 87.587203) (end 132.524033 85.957215) (width 0.7) (layer B.Cu) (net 27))
 (segment (start 112.204033 79.819967) (end 108.749999 83.274001) (width 0.7) (layer B.Cu) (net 27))
 (segment (start 121.581956 95.334044) (end 126.983752 95.334044) (width 0.7) (layer B.Cu) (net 27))
 (segment (start 130.894044 91.423752) (end 130.894044 87.587203) (width 0.7) (layer B.Cu) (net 27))
 (segment (start 132.524033 82.181186) (end 130.162814 79.819967) (width 0.7) (layer B.Cu) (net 27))
 (segment (start 108.749999 83.274001) (end 107.95 84.074) (width 0.7) (layer B.Cu) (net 27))
 (segment (start 130.162814 79.819967) (end 112.204033 79.819967) (width 0.7) (layer B.Cu) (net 27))
 (segment (start 120.142 96.774) (end 121.581956 95.334044) (width 0.7) (layer B.Cu) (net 27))
 (segment (start 105.41 84.074) (end 110.574044 78.909956) (width 0.7) (layer B.Cu) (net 28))
 (segment (start 130.539752 78.909956) (end 133.434044 81.804248) (width 0.7) (layer B.Cu) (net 28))
 (segment (start 133.434044 81.804248) (end 133.434044 86.529956) (width 0.7) (layer B.Cu) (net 28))
 (segment (start 110.574044 78.909956) (end 130.539752 78.909956) (width 0.7) (layer B.Cu) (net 28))
 (segment (start 133.434044 86.529956) (end 131.804055 88.159945) (width 0.7) (layer B.Cu) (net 28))
 (segment (start 131.804055 88.159945) (end 131.804055 91.80069) (width 0.7) (layer B.Cu) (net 28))
 (segment (start 131.804055 91.80069) (end 126.830745 96.774) (width 0.7) (layer B.Cu) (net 28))
 (segment (start 126.830745 96.774) (end 122.682 96.774) (width 0.7) (layer B.Cu) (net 28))
 (segment (start 108.144011 72.584011) (end 144.466011 72.584011) (width 1) (layer B.Cu) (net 16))
 (segment (start 103.886 68.326) (end 108.144011 72.584011) (width 1) (layer B.Cu) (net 16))
 (segment (start 144.466011 72.584011) (end 151.638 79.756) (width 1) (layer B.Cu) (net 16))
 (segment (start 105.156 65.532) (end 101.6 65.532) (width 1) (layer B.Cu) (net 15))
 (segment (start 110.998 71.374) (end 105.156 65.532) (width 1) (layer B.Cu) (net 15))
 (segment (start 101.6 65.532) (end 98.806 68.326) (width 1) (layer B.Cu) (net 15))
 (segment (start 151.638 72.136) (end 150.876 71.374) (width 1) (layer B.Cu) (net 15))
 (segment (start 150.876 71.374) (end 110.998 71.374) (width 1) (layer B.Cu) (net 15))
 (segment (start 119.329999 87.071999) (end 94.691999 87.071999) (width 0.7) (layer B.Cu) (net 33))
 (segment (start 120.65 88.392) (end 119.329999 87.071999) (width 0.7) (layer B.Cu) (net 33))
 (segment (start 120.65 89.154) (end 120.65 88.392) (width 0.7) (layer B.Cu) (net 33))
 (segment (start 87.63 70.44732) (end 87.63 68.326) (width 0.7) (layer B.Cu) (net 33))
 (segment (start 87.63 82.296) (end 87.63 70.44732) (width 0.7) (layer B.Cu) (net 33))
 (segment (start 92.405999 87.071999) (end 87.63 82.296) (width 0.7) (layer B.Cu) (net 33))
 (segment (start 94.488 87.071999) (end 92.405999 87.071999) (width 0.7) (layer B.Cu) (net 33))
 (segment (start 151.384 89.916) (end 151.638 89.916) (width 1) (layer F.Cu) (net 17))
 (segment (start 121.964011 80.308011) (end 118.11 76.454) (width 1) (layer F.Cu) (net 17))
 (segment (start 129.838011 80.308011) (end 121.964011 80.308011) (width 1) (layer F.Cu) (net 17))
 (segment (start 139.446 89.916) (end 129.838011 80.308011) (width 1) (layer F.Cu) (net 17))
 (segment (start 151.638 89.916) (end 139.446 89.916) (width 1) (layer F.Cu) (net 17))
 (segment (start 113.03 84.074) (end 113.284 84.074) (width 1) (layer B.Cu) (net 2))
 (segment (start 76.962 78.136) (end 77.058 78.232) (width 1) (layer B.Cu) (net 2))
 (segment (start 76.962 73.914) (end 76.962 78.136) (width 1) (layer B.Cu) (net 2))
 (segment (start 82.55 68.326) (end 76.962 73.914) (width 1) (layer B.Cu) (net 2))
 (segment (start 87.804 90.932) (end 89.114 89.622) (width 1) (layer B.Cu) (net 2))
 (segment (start 82.042 90.932) (end 87.804 90.932) (width 1) (layer B.Cu) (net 2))
 (segment (start 82.042 90.932) (end 84.201 93.091) (width 1) (layer B.Cu) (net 2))
 (segment (start 89.114 93.091) (end 84.201 93.091) (width 1) (layer B.Cu) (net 2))
 (segment (start 147.066 78.152) (end 147.066 66.04) (width 1) (layer F.Cu) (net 2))
 (segment (start 144.018 81.2) (end 147.066 78.152) (width 1) (layer F.Cu) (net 2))
 (segment (start 144.018 84.836) (end 151.638 92.456) (width 1) (layer B.Cu) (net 2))
 (segment (start 144.018 81.2) (end 144.018 84.836) (width 1) (layer B.Cu) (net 2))
 (segment (start 112.054 89.408) (end 113.03 88.432) (width 1) (layer F.Cu) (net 2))
 (segment (start 97.282 89.408) (end 112.054 89.408) (width 1) (layer F.Cu) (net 2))
 (segment (start 113.03 88.432) (end 113.03 84.074) (width 1) (layer F.Cu) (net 2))
 (segment (start 133.35 86.868) (end 133.35 89.154) (width 1) (layer F.Cu) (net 2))
 (segment (start 128.524 82.042) (end 133.35 86.868) (width 1) (layer F.Cu) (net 2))
 (segment (start 115.062 82.042) (end 128.524 82.042) (width 1) (layer F.Cu) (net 2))
 (segment (start 113.03 84.074) (end 115.062 82.042) (width 1) (layer F.Cu) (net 2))
 (segment (start 108.204 78.74) (end 95.25 78.74) (width 1) (layer F.Cu) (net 2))
 (segment (start 110.49 76.454) (end 108.204 78.74) (width 1) (layer F.Cu) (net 2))
 (segment (start 92.964 78.74) (end 82.55 68.326) (width 1) (layer F.Cu) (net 2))
 (segment (start 95.25 78.74) (end 92.964 78.74) (width 1) (layer F.Cu) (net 2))
 (segment (start 136.652 92.456) (end 151.638 92.456) (width 1) (layer F.Cu) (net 2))
 (segment (start 133.35 89.154) (end 136.652 92.456) (width 1) (layer F.Cu) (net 2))
 (segment (start 147.066 65.278) (end 147.066 66.294) (width 1) (layer F.Cu) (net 2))
 (segment (start 138.684 63.754) (end 145.542 63.754) (width 1) (layer F.Cu) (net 2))
 (segment (start 136.906 65.532) (end 138.684 63.754) (width 1) (layer F.Cu) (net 2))
 (segment (start 135.128 63.754) (end 136.906 65.532) (width 1) (layer F.Cu) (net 2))
 (segment (start 110.49 63.754) (end 135.128 63.754) (width 1) (layer F.Cu) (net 2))
 (segment (start 145.542 63.754) (end 147.066 65.278) (width 1) (layer F.Cu) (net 2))
 (segment (start 108.966 65.278) (end 110.49 63.754) (width 1) (layer F.Cu) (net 2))
 (segment (start 108.966 66.294) (end 108.966 65.278) (width 1) (layer F.Cu) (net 2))
 (segment (start 77.058 86.710002) (end 77.058 78.232) (width 1) (layer B.Cu) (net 2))
 (segment (start 77.058 89.472) (end 77.058 86.710002) (width 1) (layer B.Cu) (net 2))
 (segment (start 78.518 90.932) (end 77.058 89.472) (width 1) (layer B.Cu) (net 2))
 (segment (start 82.042 90.932) (end 78.518 90.932) (width 1) (layer B.Cu) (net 2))
 (segment (start 97.068 89.622) (end 97.282 89.408) (width 1) (layer B.Cu) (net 2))
 (segment (start 89.114 89.622) (end 97.068 89.622) (width 1) (layer B.Cu) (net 2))
 (segment (start 141.986 75.732) (end 139.018 78.7) (width 0.7) (layer F.Cu) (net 14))
 (segment (start 141.986 75.732) (end 141.986 66.04) (width 0.7) (layer F.Cu) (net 14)))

